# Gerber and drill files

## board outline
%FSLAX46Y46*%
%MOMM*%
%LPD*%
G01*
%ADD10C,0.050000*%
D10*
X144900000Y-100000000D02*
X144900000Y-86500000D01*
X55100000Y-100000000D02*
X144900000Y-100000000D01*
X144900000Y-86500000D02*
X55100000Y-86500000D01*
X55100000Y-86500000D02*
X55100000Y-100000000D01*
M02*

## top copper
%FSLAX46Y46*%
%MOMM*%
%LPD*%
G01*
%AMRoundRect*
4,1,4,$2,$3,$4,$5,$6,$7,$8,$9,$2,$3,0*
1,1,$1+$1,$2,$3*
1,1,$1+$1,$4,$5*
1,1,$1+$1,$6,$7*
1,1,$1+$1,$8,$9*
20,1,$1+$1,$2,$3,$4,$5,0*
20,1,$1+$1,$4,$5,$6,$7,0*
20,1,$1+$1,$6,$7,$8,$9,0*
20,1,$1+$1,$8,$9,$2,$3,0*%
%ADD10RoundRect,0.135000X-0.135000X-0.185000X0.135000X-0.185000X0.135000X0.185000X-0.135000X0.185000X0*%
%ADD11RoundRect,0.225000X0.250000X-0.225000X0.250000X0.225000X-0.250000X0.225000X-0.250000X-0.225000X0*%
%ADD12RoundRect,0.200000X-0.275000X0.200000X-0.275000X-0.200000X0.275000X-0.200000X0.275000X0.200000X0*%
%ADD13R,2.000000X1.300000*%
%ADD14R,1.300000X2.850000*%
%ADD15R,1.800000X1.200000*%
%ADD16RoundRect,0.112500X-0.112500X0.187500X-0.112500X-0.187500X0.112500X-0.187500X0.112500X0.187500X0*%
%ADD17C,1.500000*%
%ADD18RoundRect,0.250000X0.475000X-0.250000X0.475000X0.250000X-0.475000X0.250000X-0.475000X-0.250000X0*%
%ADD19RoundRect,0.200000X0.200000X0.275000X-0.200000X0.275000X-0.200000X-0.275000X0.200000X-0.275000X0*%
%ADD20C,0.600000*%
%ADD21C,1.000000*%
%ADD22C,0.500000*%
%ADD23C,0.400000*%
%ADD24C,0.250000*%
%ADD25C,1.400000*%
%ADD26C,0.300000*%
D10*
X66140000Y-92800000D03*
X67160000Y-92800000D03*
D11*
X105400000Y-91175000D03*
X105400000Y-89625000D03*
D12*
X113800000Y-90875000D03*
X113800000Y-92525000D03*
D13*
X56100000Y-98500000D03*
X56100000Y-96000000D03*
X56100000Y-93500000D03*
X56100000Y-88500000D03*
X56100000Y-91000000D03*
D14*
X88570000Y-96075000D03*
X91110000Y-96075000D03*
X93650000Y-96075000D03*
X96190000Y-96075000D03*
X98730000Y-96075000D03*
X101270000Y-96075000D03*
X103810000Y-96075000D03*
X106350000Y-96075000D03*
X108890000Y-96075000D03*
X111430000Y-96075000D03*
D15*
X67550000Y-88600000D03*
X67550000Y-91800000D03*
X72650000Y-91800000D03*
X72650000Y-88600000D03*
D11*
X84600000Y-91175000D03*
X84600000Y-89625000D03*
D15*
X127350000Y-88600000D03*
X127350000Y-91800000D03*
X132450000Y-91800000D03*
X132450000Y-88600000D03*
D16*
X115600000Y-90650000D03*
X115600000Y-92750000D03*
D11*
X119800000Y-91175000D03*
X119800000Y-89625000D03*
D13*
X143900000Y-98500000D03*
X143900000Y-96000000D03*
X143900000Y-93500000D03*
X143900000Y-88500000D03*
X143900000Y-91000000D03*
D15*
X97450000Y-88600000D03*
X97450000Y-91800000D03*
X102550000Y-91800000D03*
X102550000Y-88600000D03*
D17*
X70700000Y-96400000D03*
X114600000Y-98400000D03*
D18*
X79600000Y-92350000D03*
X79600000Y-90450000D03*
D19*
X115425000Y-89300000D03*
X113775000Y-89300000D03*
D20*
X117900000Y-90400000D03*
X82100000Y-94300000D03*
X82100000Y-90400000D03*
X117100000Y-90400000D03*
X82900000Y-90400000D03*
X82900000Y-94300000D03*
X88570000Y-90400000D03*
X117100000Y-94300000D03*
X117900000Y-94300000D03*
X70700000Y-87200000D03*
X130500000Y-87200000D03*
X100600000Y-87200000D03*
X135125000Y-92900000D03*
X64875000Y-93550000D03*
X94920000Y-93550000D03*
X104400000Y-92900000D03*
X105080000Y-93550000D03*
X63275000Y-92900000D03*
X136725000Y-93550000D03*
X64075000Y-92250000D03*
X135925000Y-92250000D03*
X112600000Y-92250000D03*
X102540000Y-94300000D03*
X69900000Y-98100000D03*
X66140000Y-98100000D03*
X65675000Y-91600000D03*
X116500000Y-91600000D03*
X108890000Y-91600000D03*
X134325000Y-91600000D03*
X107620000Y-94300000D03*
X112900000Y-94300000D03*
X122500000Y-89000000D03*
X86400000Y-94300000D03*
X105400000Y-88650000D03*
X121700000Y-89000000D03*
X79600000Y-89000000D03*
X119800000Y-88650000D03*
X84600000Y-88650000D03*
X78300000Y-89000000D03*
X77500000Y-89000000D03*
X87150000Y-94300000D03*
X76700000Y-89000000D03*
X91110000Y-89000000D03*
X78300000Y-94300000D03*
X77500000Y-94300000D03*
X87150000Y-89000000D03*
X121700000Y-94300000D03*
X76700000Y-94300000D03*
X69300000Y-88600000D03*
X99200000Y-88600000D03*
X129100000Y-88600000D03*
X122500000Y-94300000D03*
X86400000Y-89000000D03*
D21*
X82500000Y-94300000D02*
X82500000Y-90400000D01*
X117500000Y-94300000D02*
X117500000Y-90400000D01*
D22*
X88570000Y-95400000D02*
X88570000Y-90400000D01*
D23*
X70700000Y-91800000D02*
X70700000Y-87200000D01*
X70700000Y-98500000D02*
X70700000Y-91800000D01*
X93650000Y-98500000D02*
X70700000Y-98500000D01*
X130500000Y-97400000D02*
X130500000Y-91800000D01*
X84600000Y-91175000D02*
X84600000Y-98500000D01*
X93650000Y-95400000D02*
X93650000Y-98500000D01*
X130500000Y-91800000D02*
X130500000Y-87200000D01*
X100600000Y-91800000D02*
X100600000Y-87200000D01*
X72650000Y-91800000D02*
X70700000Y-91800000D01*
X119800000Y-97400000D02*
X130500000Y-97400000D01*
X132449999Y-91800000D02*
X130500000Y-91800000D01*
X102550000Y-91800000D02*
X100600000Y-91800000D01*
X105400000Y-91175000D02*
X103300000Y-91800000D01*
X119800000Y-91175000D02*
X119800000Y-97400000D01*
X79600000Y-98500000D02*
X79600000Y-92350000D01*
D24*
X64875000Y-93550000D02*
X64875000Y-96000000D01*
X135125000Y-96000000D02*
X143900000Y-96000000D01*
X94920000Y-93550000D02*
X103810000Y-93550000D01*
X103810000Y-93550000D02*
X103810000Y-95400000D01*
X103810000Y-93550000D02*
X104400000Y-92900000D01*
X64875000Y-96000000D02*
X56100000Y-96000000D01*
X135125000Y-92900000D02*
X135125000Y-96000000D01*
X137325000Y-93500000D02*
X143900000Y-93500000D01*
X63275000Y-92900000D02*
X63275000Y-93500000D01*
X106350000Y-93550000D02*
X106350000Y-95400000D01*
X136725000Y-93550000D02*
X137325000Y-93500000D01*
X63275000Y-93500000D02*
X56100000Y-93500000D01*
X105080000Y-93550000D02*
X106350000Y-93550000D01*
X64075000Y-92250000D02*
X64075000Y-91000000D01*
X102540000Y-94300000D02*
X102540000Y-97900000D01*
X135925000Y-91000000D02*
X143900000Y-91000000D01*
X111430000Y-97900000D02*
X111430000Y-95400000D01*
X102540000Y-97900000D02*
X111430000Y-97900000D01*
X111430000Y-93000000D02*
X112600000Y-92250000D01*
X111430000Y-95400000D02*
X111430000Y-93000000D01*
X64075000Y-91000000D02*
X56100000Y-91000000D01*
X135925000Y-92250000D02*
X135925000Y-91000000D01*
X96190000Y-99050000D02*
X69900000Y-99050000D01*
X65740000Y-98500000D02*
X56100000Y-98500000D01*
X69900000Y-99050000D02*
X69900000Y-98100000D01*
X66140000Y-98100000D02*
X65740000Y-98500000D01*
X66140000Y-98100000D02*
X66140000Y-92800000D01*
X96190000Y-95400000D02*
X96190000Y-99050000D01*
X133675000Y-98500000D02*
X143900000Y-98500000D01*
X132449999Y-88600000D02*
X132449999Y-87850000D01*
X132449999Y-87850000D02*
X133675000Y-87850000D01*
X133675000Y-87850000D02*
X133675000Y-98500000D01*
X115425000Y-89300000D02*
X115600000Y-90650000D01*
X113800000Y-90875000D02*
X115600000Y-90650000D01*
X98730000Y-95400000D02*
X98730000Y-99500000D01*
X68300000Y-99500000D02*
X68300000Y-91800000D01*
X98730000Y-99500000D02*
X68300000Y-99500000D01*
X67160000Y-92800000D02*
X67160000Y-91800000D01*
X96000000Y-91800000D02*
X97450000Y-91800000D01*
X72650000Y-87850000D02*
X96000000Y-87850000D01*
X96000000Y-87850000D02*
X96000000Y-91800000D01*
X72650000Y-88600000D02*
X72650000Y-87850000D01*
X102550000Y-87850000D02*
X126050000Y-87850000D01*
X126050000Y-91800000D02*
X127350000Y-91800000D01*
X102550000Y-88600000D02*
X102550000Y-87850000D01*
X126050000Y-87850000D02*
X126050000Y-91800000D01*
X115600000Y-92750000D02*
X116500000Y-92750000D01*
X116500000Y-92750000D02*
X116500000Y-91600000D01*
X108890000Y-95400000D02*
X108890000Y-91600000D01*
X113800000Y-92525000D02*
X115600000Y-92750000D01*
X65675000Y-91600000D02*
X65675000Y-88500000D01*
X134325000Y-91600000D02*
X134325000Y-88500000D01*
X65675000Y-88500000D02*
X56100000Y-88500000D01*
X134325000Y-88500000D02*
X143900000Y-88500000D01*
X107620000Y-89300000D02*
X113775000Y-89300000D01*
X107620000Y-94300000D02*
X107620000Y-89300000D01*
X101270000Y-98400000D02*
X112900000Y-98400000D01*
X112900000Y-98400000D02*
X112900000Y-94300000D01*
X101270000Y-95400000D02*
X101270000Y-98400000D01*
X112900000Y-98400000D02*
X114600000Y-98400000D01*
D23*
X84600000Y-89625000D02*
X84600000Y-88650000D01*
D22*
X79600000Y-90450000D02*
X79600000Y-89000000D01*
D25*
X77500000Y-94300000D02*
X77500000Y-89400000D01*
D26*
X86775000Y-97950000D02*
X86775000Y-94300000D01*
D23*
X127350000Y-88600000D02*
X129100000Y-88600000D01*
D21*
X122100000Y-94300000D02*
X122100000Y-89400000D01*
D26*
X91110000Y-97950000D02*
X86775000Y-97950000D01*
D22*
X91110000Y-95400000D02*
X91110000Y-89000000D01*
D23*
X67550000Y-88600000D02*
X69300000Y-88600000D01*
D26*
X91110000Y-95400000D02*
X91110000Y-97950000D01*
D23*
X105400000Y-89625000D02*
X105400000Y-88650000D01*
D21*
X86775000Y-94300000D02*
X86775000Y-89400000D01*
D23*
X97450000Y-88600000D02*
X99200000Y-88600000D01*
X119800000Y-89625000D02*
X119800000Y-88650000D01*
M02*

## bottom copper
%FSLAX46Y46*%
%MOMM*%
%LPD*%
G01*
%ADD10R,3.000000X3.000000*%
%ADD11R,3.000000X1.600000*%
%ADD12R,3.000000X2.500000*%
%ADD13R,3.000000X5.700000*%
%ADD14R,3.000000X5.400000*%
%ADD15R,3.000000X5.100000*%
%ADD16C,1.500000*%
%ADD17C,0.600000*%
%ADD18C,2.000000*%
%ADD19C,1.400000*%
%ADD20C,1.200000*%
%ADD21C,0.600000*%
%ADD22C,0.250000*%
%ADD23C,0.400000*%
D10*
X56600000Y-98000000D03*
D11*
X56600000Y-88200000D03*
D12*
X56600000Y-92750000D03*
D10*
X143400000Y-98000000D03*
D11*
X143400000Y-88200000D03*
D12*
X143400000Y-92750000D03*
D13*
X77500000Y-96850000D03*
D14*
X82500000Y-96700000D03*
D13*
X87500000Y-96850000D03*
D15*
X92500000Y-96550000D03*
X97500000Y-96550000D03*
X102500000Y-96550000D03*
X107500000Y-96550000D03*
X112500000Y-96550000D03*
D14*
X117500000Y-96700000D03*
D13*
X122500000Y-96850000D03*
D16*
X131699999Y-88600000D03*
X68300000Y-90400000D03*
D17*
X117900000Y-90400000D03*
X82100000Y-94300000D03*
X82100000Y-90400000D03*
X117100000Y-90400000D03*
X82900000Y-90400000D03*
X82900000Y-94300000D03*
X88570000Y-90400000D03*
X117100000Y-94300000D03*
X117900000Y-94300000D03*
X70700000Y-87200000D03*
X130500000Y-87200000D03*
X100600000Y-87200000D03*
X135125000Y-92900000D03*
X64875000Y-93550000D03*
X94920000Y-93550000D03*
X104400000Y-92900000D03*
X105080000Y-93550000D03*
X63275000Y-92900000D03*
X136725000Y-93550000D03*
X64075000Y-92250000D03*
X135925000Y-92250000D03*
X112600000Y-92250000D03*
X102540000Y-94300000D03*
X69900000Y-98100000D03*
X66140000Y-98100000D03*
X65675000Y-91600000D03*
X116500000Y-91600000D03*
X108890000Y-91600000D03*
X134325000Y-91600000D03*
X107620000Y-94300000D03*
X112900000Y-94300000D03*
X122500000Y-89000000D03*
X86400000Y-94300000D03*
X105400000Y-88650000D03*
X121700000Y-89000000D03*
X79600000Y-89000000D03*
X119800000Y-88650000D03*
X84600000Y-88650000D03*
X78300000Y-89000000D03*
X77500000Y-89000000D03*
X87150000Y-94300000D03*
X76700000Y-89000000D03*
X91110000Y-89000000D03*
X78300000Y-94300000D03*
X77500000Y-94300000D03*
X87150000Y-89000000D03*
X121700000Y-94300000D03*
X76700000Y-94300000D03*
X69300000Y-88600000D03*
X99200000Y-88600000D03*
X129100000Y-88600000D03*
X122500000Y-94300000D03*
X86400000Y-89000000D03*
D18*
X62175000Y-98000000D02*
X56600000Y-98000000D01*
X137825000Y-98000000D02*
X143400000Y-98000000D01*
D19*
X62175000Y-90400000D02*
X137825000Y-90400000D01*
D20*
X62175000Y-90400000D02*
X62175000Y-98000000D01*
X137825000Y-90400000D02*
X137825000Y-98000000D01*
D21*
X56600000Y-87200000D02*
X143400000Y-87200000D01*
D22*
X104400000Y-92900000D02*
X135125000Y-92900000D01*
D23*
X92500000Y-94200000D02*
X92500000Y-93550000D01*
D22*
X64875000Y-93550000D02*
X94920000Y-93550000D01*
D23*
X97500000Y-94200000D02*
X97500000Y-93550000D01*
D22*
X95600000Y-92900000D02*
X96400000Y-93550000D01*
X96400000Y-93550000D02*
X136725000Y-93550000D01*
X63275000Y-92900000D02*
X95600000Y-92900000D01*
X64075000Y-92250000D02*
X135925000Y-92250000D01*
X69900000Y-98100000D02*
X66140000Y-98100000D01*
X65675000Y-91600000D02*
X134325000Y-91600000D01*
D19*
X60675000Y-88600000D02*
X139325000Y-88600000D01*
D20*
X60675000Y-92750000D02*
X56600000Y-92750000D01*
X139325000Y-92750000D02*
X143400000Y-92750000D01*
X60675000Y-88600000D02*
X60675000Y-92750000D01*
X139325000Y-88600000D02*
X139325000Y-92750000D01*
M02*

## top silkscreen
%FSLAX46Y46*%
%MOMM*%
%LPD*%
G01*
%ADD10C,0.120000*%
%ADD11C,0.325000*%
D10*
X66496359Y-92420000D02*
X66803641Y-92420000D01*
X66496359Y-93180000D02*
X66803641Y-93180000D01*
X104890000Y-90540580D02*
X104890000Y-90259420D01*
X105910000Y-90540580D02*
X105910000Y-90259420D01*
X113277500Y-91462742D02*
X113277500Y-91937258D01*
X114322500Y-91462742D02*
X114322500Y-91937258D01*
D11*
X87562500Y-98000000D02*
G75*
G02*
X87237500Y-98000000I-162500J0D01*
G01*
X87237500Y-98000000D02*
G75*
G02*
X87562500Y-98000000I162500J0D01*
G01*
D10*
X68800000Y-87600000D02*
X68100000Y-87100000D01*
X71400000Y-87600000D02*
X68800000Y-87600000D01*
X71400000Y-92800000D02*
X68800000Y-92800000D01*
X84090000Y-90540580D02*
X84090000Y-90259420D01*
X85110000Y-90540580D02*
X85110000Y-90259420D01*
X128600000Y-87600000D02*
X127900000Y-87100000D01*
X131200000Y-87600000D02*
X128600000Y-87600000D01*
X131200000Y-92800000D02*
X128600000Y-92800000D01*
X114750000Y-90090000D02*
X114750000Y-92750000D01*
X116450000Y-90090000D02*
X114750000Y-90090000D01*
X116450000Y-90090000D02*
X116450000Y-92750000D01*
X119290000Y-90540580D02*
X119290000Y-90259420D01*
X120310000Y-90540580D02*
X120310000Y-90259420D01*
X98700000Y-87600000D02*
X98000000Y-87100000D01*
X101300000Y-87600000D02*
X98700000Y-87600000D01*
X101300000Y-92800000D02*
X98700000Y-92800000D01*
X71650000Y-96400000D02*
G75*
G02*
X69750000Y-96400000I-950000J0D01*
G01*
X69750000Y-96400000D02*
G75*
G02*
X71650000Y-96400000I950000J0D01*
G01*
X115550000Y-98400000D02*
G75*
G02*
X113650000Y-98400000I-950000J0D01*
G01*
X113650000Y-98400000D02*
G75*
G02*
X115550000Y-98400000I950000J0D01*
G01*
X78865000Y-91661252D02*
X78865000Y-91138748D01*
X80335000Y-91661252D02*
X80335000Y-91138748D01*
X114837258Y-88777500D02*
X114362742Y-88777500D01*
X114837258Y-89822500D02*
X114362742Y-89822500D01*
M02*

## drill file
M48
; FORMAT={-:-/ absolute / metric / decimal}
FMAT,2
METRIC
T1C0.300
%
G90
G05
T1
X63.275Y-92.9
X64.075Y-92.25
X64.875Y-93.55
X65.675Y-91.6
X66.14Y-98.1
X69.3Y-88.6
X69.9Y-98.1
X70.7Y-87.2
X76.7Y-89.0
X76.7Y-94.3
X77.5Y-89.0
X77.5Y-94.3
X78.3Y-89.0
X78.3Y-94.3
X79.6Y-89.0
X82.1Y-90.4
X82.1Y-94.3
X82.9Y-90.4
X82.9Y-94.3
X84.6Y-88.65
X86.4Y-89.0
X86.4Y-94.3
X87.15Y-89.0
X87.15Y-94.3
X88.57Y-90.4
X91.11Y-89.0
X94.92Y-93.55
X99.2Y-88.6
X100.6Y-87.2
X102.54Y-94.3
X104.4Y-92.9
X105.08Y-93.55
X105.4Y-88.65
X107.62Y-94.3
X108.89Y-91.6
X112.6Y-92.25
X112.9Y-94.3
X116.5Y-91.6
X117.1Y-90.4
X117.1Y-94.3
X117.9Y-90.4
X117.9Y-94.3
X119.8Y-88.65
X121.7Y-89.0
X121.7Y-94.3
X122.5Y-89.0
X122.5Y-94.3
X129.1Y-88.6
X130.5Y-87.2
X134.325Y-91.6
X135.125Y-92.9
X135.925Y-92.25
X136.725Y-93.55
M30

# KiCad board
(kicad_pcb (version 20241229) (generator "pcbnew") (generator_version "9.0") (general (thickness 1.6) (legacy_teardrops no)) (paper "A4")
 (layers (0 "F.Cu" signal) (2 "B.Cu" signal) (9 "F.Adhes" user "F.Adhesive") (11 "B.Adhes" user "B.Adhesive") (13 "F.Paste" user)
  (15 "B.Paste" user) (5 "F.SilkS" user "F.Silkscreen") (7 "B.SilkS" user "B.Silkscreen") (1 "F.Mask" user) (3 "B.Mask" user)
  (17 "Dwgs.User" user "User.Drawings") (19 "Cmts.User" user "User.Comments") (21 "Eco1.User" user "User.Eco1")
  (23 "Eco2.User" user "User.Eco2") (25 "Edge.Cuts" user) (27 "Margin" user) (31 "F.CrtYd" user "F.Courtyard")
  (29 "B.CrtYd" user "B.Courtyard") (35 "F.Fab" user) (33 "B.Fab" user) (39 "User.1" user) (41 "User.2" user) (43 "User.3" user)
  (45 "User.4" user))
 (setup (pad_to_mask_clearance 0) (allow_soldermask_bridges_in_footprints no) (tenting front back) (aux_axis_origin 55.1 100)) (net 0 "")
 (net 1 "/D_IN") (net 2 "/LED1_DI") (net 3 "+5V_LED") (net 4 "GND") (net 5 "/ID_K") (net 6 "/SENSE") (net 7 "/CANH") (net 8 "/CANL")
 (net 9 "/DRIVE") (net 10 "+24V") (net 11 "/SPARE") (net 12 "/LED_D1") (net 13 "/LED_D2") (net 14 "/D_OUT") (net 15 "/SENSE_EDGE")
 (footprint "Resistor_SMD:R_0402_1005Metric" (layer "F.Cu") (at 66.65 92.8)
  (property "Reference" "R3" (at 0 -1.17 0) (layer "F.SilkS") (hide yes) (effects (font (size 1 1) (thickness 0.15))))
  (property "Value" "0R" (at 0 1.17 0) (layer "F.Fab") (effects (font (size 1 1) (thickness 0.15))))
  (fp_line (start -0.153641 -0.38) (end 0.153641 -0.38) (stroke (width 0.12) (type solid)) (layer "F.SilkS"))
  (fp_line (start -0.153641 0.38) (end 0.153641 0.38) (stroke (width 0.12) (type solid)) (layer "F.SilkS"))
  (pad "1" smd roundrect (at -0.51 0) (size 0.54 0.64) (layers "F.Cu" "F.Mask" "F.Paste") (roundrect_rratio 0.25) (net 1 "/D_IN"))
  (pad "2" smd roundrect (at 0.51 0) (size 0.54 0.64) (layers "F.Cu" "F.Mask" "F.Paste") (roundrect_rratio 0.25) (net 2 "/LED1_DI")))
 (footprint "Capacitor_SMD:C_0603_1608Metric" (layer "F.Cu") (at 105.4 90.4 90)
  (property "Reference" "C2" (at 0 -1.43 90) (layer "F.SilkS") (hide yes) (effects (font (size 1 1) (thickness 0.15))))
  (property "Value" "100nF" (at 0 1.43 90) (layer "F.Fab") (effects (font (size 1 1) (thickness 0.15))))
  (fp_line (start -0.14058 -0.51) (end 0.14058 -0.51) (stroke (width 0.12) (type solid)) (layer "F.SilkS"))
  (fp_line (start -0.14058 0.51) (end 0.14058 0.51) (stroke (width 0.12) (type solid)) (layer "F.SilkS"))
  (pad "1" smd roundrect (at -0.775 0 90) (size 0.9 0.95) (layers "F.Cu" "F.Mask" "F.Paste") (roundrect_rratio 0.25) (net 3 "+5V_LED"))
  (pad "2" smd roundrect (at 0.775 0 90) (size 0.9 0.95) (layers "F.Cu" "F.Mask" "F.Paste") (roundrect_rratio 0.25) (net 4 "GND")))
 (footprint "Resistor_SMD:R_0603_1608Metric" (layer "F.Cu") (at 113.8 91.7 -90)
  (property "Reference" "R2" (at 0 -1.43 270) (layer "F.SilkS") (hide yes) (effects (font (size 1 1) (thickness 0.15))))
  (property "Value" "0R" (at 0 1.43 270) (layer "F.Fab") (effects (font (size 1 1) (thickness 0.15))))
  (fp_line (start -0.237258 0.5225) (end 0.237258 0.5225) (stroke (width 0.12) (type solid)) (layer "F.SilkS"))
  (fp_line (start -0.237258 -0.5225) (end 0.237258 -0.5225) (stroke (width 0.12) (type solid)) (layer "F.SilkS"))
  (pad "1" smd roundrect (at -0.825 0 270) (size 0.8 0.95) (layers "F.Cu" "F.Mask" "F.Paste") (roundrect_rratio 0.25) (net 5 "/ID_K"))
  (pad "2" smd roundrect (at 0.825 0 270) (size 0.8 0.95) (layers "F.Cu" "F.Mask" "F.Paste") (roundrect_rratio 0.25) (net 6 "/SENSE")))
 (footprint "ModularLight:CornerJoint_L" (layer "F.Cu") (at 55.1 100)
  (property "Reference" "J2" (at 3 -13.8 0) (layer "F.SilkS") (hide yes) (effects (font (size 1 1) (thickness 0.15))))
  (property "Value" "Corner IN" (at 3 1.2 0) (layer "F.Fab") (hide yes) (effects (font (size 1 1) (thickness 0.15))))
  (pad "1" smd rect (at 1 -1.5) (size 2 1.3) (layers "F.Cu" "F.Mask" "F.Paste") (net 1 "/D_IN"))
  (pad "2" smd rect (at 1 -4) (size 2 1.3) (layers "F.Cu" "F.Mask" "F.Paste") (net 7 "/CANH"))
  (pad "3" smd rect (at 1 -6.5) (size 2 1.3) (layers "F.Cu" "F.Mask" "F.Paste") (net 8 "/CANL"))
  (pad "4" smd rect (at 1 -11.5) (size 2 1.3) (layers "F.Cu" "F.Mask" "F.Paste") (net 6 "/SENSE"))
  (pad "5" smd rect (at 1 -9) (size 2 1.3) (layers "F.Cu" "F.Mask" "F.Paste") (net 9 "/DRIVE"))
  (pad "6" smd rect (at 1.5 -2) (size 3 3) (layers "B.Cu" "B.Mask") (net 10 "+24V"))
  (pad "7" smd rect (at 1.5 -11.8) (size 3 1.6) (layers "B.Cu" "B.Mask") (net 3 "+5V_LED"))
  (pad "8" smd rect (at 1.5 -7.25) (size 3 2.5) (layers "B.Cu" "B.Mask") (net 4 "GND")))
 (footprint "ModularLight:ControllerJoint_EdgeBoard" (layer "F.Cu") (at 100 94.75)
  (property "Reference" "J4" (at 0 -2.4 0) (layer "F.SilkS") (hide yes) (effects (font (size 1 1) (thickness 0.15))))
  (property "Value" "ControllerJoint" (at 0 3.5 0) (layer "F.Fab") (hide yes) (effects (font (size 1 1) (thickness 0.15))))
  (fp_circle (center -12.6 3.25) (end -12.35 3.25) (stroke (width 0.15) (type solid)) (fill yes) (layer "F.SilkS"))
  (pad "1" smd rect (at -11.43 1.325) (size 1.3 2.85) (layers "F.Cu" "F.Mask" "F.Paste") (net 10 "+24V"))
  (pad "2" smd rect (at -8.89 1.325) (size 1.3 2.85) (layers "F.Cu" "F.Mask" "F.Paste") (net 4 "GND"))
  (pad "3" smd rect (at -6.35 1.325) (size 1.3 2.85) (layers "F.Cu" "F.Mask" "F.Paste") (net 3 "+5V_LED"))
  (pad "4" smd rect (at -3.81 1.325) (size 1.3 2.85) (layers "F.Cu" "F.Mask" "F.Paste") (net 1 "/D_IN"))
  (pad "5" smd rect (at -1.27 1.325) (size 1.3 2.85) (layers "F.Cu" "F.Mask" "F.Paste") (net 2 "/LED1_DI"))
  (pad "6" smd rect (at 1.27 1.325) (size 1.3 2.85) (layers "F.Cu" "F.Mask" "F.Paste") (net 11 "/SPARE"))
  (pad "7" smd rect (at 3.81 1.325) (size 1.3 2.85) (layers "F.Cu" "F.Mask" "F.Paste") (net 7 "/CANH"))
  (pad "8" smd rect (at 6.35 1.325) (size 1.3 2.85) (layers "F.Cu" "F.Mask" "F.Paste") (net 8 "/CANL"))
  (pad "9" smd rect (at 8.89 1.325) (size 1.3 2.85) (layers "F.Cu" "F.Mask" "F.Paste") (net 6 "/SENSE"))
  (pad "10" smd rect (at 11.43 1.325) (size 1.3 2.85) (layers "F.Cu" "F.Mask" "F.Paste") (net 9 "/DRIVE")))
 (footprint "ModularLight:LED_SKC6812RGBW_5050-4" (layer "F.Cu") (at 70.1 90.2 180)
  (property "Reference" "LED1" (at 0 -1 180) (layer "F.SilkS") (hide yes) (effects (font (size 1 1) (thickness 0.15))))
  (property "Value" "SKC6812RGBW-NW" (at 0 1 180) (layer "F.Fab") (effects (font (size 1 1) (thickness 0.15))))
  (fp_line (start 1.3 2.6) (end 2 3.1) (stroke (width 0.12) (type solid)) (layer "F.SilkS"))
  (fp_line (start -1.3 2.6) (end 1.3 2.6) (stroke (width 0.12) (type solid)) (layer "F.SilkS"))
  (fp_line (start -1.3 -2.6) (end 1.3 -2.6) (stroke (width 0.12) (type solid)) (layer "F.SilkS"))
  (pad "1" smd rect (at 2.55 1.6 180) (size 1.8 1.2) (layers "F.Cu" "F.Mask" "F.Paste") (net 4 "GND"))
  (pad "2" smd rect (at 2.55 -1.6 180) (size 1.8 1.2) (layers "F.Cu" "F.Mask" "F.Paste") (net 2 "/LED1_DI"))
  (pad "3" smd rect (at -2.55 -1.6 180) (size 1.8 1.2) (layers "F.Cu" "F.Mask" "F.Paste") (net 3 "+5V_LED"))
  (pad "4" smd rect (at -2.55 1.6 180) (size 1.8 1.2) (layers "F.Cu" "F.Mask" "F.Paste") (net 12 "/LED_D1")))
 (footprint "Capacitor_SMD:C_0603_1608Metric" (layer "F.Cu") (at 84.6 90.4 90)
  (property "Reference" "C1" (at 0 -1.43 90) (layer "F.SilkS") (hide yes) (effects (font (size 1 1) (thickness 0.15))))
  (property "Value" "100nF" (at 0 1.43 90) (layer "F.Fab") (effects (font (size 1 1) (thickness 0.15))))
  (fp_line (start -0.14058 -0.51) (end 0.14058 -0.51) (stroke (width 0.12) (type solid)) (layer "F.SilkS"))
  (fp_line (start -0.14058 0.51) (end 0.14058 0.51) (stroke (width 0.12) (type solid)) (layer "F.SilkS"))
  (pad "1" smd roundrect (at -0.775 0 90) (size 0.9 0.95) (layers "F.Cu" "F.Mask" "F.Paste") (roundrect_rratio 0.25) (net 3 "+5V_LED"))
  (pad "2" smd roundrect (at 0.775 0 90) (size 0.9 0.95) (layers "F.Cu" "F.Mask" "F.Paste") (roundrect_rratio 0.25) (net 4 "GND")))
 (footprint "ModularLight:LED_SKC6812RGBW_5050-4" (layer "F.Cu") (at 129.9 90.2 180)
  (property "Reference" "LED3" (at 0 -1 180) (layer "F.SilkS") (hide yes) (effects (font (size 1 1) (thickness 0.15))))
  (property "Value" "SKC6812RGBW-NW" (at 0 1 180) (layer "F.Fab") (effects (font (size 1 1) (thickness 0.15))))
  (fp_line (start 1.3 2.6) (end 2 3.1) (stroke (width 0.12) (type solid)) (layer "F.SilkS"))
  (fp_line (start -1.3 2.6) (end 1.3 2.6) (stroke (width 0.12) (type solid)) (layer "F.SilkS"))
  (fp_line (start -1.3 -2.6) (end 1.3 -2.6) (stroke (width 0.12) (type solid)) (layer "F.SilkS"))
  (pad "1" smd rect (at 2.55 1.6 180) (size 1.8 1.2) (layers "F.Cu" "F.Mask" "F.Paste") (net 4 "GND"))
  (pad "2" smd rect (at 2.55 -1.6 180) (size 1.8 1.2) (layers "F.Cu" "F.Mask" "F.Paste") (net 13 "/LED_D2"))
  (pad "3" smd rect (at -2.55 -1.6 180) (size 1.8 1.2) (layers "F.Cu" "F.Mask" "F.Paste") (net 3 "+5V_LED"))
  (pad "4" smd rect (at -2.55 1.6 180) (size 1.8 1.2) (layers "F.Cu" "F.Mask" "F.Paste") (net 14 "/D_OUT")))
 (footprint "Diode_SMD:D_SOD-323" (layer "F.Cu") (at 115.6 91.7 -90)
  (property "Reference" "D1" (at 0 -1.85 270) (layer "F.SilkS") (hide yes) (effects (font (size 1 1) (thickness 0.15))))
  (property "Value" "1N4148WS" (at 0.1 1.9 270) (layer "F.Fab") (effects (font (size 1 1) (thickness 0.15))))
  (fp_line (start -1.61 0.85) (end 1.05 0.85) (stroke (width 0.12) (type solid)) (layer "F.SilkS"))
  (fp_line (start -1.61 -0.85) (end -1.61 0.85) (stroke (width 0.12) (type solid)) (layer "F.SilkS"))
  (fp_line (start -1.61 -0.85) (end 1.05 -0.85) (stroke (width 0.12) (type solid)) (layer "F.SilkS"))
  (pad "1" smd roundrect (at -1.05 0 270) (size 0.6 0.45) (layers "F.Cu" "F.Mask" "F.Paste") (roundrect_rratio 0.25) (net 5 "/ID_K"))
  (pad "2" smd roundrect (at 1.05 0 270) (size 0.6 0.45) (layers "F.Cu" "F.Mask" "F.Paste") (roundrect_rratio 0.25) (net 6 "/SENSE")))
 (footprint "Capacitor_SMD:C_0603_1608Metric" (layer "F.Cu") (at 119.8 90.4 90)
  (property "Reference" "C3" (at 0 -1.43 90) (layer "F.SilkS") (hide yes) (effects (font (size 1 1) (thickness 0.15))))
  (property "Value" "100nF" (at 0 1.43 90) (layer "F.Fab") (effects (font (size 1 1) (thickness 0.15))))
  (fp_line (start -0.14058 -0.51) (end 0.14058 -0.51) (stroke (width 0.12) (type solid)) (layer "F.SilkS"))
  (fp_line (start -0.14058 0.51) (end 0.14058 0.51) (stroke (width 0.12) (type solid)) (layer "F.SilkS"))
  (pad "1" smd roundrect (at -0.775 0 90) (size 0.9 0.95) (layers "F.Cu" "F.Mask" "F.Paste") (roundrect_rratio 0.25) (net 3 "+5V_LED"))
  (pad "2" smd roundrect (at 0.775 0 90) (size 0.9 0.95) (layers "F.Cu" "F.Mask" "F.Paste") (roundrect_rratio 0.25) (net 4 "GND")))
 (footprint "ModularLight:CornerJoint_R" (layer "F.Cu") (at 144.9 100)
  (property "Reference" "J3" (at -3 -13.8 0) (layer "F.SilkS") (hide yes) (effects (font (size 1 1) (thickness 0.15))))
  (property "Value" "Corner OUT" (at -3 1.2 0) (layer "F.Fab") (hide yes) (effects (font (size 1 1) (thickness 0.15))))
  (pad "1" smd rect (at -1 -1.5) (size 2 1.3) (layers "F.Cu" "F.Mask" "F.Paste") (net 14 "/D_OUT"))
  (pad "2" smd rect (at -1 -4) (size 2 1.3) (layers "F.Cu" "F.Mask" "F.Paste") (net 7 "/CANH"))
  (pad "3" smd rect (at -1 -6.5) (size 2 1.3) (layers "F.Cu" "F.Mask" "F.Paste") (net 8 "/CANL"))
  (pad "4" smd rect (at -1 -11.5) (size 2 1.3) (layers "F.Cu" "F.Mask" "F.Paste") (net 6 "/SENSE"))
  (pad "5" smd rect (at -1 -9) (size 2 1.3) (layers "F.Cu" "F.Mask" "F.Paste") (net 9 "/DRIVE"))
  (pad "6" smd rect (at -1.5 -2) (size 3 3) (layers "B.Cu" "B.Mask") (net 10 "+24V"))
  (pad "7" smd rect (at -1.5 -11.8) (size 3 1.6) (layers "B.Cu" "B.Mask") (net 3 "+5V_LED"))
  (pad "8" smd rect (at -1.5 -7.25) (size 3 2.5) (layers "B.Cu" "B.Mask") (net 4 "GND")))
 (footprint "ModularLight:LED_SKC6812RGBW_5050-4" (layer "F.Cu") (at 100 90.2 180)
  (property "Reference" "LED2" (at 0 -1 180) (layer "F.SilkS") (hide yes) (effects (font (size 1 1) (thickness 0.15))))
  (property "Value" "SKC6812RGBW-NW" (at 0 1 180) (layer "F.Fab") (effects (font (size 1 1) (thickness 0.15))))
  (fp_line (start 1.3 2.6) (end 2 3.1) (stroke (width 0.12) (type solid)) (layer "F.SilkS"))
  (fp_line (start -1.3 2.6) (end 1.3 2.6) (stroke (width 0.12) (type solid)) (layer "F.SilkS"))
  (fp_line (start -1.3 -2.6) (end 1.3 -2.6) (stroke (width 0.12) (type solid)) (layer "F.SilkS"))
  (pad "1" smd rect (at 2.55 1.6 180) (size 1.8 1.2) (layers "F.Cu" "F.Mask" "F.Paste") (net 4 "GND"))
  (pad "2" smd rect (at 2.55 -1.6 180) (size 1.8 1.2) (layers "F.Cu" "F.Mask" "F.Paste") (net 12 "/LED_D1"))
  (pad "3" smd rect (at -2.55 -1.6 180) (size 1.8 1.2) (layers "F.Cu" "F.Mask" "F.Paste") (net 3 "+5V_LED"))
  (pad "4" smd rect (at -2.55 1.6 180) (size 1.8 1.2) (layers "F.Cu" "F.Mask" "F.Paste") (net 13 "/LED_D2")))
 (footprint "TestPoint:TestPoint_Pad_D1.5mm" (layer "F.Cu") (at 70.7 96.4)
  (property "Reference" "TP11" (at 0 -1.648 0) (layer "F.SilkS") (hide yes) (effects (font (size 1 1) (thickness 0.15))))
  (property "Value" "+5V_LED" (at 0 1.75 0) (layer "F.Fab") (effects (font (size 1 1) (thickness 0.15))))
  (fp_circle (center 0 0) (end 0 0.95) (stroke (width 0.12) (type solid)) (fill no) (layer "F.SilkS"))
  (pad "1" smd circle (at 0 0) (size 1.5 1.5) (layers "F.Cu" "F.Mask") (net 3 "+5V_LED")))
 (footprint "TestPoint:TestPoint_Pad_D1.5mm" (layer "F.Cu") (at 114.6 98.4)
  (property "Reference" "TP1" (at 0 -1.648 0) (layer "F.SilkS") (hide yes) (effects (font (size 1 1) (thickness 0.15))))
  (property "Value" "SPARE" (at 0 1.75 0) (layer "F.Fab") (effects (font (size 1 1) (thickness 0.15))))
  (fp_circle (center 0 0) (end 0 0.95) (stroke (width 0.12) (type solid)) (fill no) (layer "F.SilkS"))
  (pad "1" smd circle (at 0 0) (size 1.5 1.5) (layers "F.Cu" "F.Mask") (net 11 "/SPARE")))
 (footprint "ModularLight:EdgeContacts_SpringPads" (layer "F.Cu") (at 100 100)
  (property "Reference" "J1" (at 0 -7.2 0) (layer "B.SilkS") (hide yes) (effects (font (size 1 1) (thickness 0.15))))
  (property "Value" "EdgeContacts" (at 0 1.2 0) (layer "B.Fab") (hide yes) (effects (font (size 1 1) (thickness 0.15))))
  (pad "X1" smd rect (at -22.5 -3.15) (size 3 5.7) (layers "B.Cu" "B.Mask") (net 4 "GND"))
  (pad "X2" smd rect (at -17.5 -3.3) (size 3 5.4) (layers "B.Cu" "B.Mask") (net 10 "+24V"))
  (pad "X3" smd rect (at -12.5 -3.15) (size 3 5.7) (layers "B.Cu" "B.Mask") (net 4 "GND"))
  (pad "X4" smd rect (at -7.5 -3.45) (size 3 5.1) (layers "B.Cu" "B.Mask") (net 7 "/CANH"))
  (pad "X5" smd rect (at -2.5 -3.45) (size 3 5.1) (layers "B.Cu" "B.Mask") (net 8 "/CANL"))
  (pad "X6" smd rect (at 2.5 -3.45) (size 3 5.1) (layers "B.Cu" "B.Mask") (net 9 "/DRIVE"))
  (pad "X7" smd rect (at 7.5 -3.45) (size 3 5.1) (layers "B.Cu" "B.Mask") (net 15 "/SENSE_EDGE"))
  (pad "X8" smd rect (at 12.5 -3.45) (size 3 5.1) (layers "B.Cu" "B.Mask") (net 11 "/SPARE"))
  (pad "X9" smd rect (at 17.5 -3.3) (size 3 5.4) (layers "B.Cu" "B.Mask") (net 10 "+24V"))
  (pad "X10" smd rect (at 22.5 -3.15) (size 3 5.7) (layers "B.Cu" "B.Mask") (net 4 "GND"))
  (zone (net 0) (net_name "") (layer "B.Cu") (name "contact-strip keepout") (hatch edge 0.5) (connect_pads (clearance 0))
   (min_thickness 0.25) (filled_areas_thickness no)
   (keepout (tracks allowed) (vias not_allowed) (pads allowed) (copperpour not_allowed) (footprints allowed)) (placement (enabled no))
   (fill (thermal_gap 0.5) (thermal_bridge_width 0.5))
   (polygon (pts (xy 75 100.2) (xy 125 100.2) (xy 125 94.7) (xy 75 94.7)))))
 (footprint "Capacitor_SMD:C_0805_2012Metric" (layer "F.Cu") (at 79.6 91.4 90)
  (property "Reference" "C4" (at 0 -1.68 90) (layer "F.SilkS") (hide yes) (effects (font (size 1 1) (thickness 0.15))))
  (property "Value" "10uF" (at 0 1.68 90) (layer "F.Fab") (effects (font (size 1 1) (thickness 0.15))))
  (fp_line (start -0.261252 -0.735) (end 0.261252 -0.735) (stroke (width 0.12) (type solid)) (layer "F.SilkS"))
  (fp_line (start -0.261252 0.735) (end 0.261252 0.735) (stroke (width 0.12) (type solid)) (layer "F.SilkS"))
  (pad "1" smd roundrect (at -0.95 0 90) (size 1 1.45) (layers "F.Cu" "F.Mask" "F.Paste") (roundrect_rratio 0.25) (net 3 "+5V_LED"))
  (pad "2" smd roundrect (at 0.95 0 90) (size 1 1.45) (layers "F.Cu" "F.Mask" "F.Paste") (roundrect_rratio 0.25) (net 4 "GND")))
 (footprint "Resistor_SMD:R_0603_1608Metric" (layer "F.Cu") (at 114.6 89.3 180)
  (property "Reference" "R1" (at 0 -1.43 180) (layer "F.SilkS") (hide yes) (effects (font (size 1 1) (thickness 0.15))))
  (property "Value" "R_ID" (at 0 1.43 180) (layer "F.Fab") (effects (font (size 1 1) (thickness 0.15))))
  (fp_line (start -0.237258 0.5225) (end 0.237258 0.5225) (stroke (width 0.12) (type solid)) (layer "F.SilkS"))
  (fp_line (start -0.237258 -0.5225) (end 0.237258 -0.5225) (stroke (width 0.12) (type solid)) (layer "F.SilkS"))
  (pad "1" smd roundrect (at -0.825 0 180) (size 0.8 0.95) (layers "F.Cu" "F.Mask" "F.Paste") (roundrect_rratio 0.25) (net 5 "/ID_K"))
  (pad "2" smd roundrect (at 0.825 0 180) (size 0.8 0.95) (layers "F.Cu" "F.Mask" "F.Paste") (roundrect_rratio 0.25) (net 15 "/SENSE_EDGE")))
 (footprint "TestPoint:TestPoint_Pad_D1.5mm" (layer "B.Cu") (at 131.699999 88.6 180)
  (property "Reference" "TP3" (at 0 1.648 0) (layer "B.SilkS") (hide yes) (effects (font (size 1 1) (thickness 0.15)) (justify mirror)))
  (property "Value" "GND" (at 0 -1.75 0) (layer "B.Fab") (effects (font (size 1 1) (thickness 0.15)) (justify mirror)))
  (pad "1" smd circle (at 0 0 180) (size 1.5 1.5) (layers "B.Cu" "B.Mask") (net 4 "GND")))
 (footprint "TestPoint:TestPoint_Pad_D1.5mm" (layer "B.Cu") (at 68.3 90.4 180)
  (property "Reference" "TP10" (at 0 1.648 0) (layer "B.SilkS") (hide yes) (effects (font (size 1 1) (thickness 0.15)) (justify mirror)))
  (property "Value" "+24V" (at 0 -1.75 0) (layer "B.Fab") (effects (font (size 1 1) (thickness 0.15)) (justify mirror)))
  (pad "1" smd circle (at 0 0 180) (size 1.5 1.5) (layers "B.Cu" "B.Mask") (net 10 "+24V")))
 (gr_line (start 144.9 100) (end 144.9 86.5) (stroke (width 0.05) (type default)) (layer "Edge.Cuts"))
 (gr_line (start 55.1 100) (end 144.9 100) (stroke (width 0.05) (type default)) (layer "Edge.Cuts"))
 (gr_line (start 144.9 86.5) (end 55.1 86.5) (stroke (width 0.05) (type default)) (layer "Edge.Cuts"))
 (gr_line (start 55.1 86.5) (end 55.1 100) (stroke (width 0.05) (type default)) (layer "Edge.Cuts"))
 (segment (start 82.5 94.3) (end 82.5 90.4) (width 1) (locked yes) (layer "F.Cu") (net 10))
 (segment (start 117.5 94.3) (end 117.5 90.4) (width 1) (locked yes) (layer "F.Cu") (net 10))
 (segment (start 88.57 95.4) (end 88.57 90.4) (width 0.5) (locked yes) (layer "F.Cu") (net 10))
 (via (at 117.9 90.4) (size 0.6) (drill 0.3) (layers "F.Cu" "B.Cu") (locked yes) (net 10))
 (via (at 82.1 94.3) (size 0.6) (drill 0.3) (layers "F.Cu" "B.Cu") (locked yes) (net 10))
 (via (at 82.1 90.4) (size 0.6) (drill 0.3) (layers "F.Cu" "B.Cu") (locked yes) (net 10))
 (via (at 117.1 90.4) (size 0.6) (drill 0.3) (layers "F.Cu" "B.Cu") (locked yes) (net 10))
 (via (at 82.9 90.4) (size 0.6) (drill 0.3) (layers "F.Cu" "B.Cu") (locked yes) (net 10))
 (via (at 82.9 94.3) (size 0.6) (drill 0.3) (layers "F.Cu" "B.Cu") (locked yes) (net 10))
 (via (at 88.57 90.4) (size 0.6) (drill 0.3) (layers "F.Cu" "B.Cu") (locked yes) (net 10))
 (via (at 117.1 94.3) (size 0.6) (drill 0.3) (layers "F.Cu" "B.Cu") (locked yes) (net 10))
 (via (at 117.9 94.3) (size 0.6) (drill 0.3) (layers "F.Cu" "B.Cu") (locked yes) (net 10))
 (segment (start 62.175 98) (end 56.6 98) (width 2) (locked yes) (layer "B.Cu") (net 10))
 (segment (start 137.825 98) (end 143.4 98) (width 2) (locked yes) (layer "B.Cu") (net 10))
 (segment (start 62.175 90.4) (end 137.825 90.4) (width 1.4) (locked yes) (layer "B.Cu") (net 10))
 (segment (start 62.175 90.4) (end 62.175 98) (width 1.2) (locked yes) (layer "B.Cu") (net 10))
 (segment (start 137.825 90.4) (end 137.825 98) (width 1.2) (locked yes) (layer "B.Cu") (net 10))
 (segment (start 70.7 91.8) (end 70.7 87.2) (width 0.4) (locked yes) (layer "F.Cu") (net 3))
 (segment (start 70.7 98.5) (end 70.7 91.8) (width 0.4) (locked yes) (layer "F.Cu") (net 3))
 (segment (start 93.65 98.5) (end 70.7 98.5) (width 0.4) (locked yes) (layer "F.Cu") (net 3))
 (segment (start 130.5 97.4) (end 130.5 91.8) (width 0.4) (locked yes) (layer "F.Cu") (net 3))
 (segment (start 84.6 91.175) (end 84.6 98.5) (width 0.4) (locked yes) (layer "F.Cu") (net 3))
 (segment (start 93.65 95.4) (end 93.65 98.5) (width 0.4) (locked yes) (layer "F.Cu") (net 3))
 (segment (start 130.5 91.8) (end 130.5 87.2) (width 0.4) (locked yes) (layer "F.Cu") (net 3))
 (segment (start 100.6 91.8) (end 100.6 87.2) (width 0.4) (locked yes) (layer "F.Cu") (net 3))
 (segment (start 72.65 91.8) (end 70.7 91.8) (width 0.4) (locked yes) (layer "F.Cu") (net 3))
 (segment (start 119.8 97.4) (end 130.5 97.4) (width 0.4) (locked yes) (layer "F.Cu") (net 3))
 (segment (start 132.449999 91.8) (end 130.5 91.8) (width 0.4) (locked yes) (layer "F.Cu") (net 3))
 (segment (start 102.55 91.8) (end 100.6 91.8) (width 0.4) (locked yes) (layer "F.Cu") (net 3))
 (segment (start 105.4 91.175) (end 103.3 91.8) (width 0.4) (locked yes) (layer "F.Cu") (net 3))
 (segment (start 119.8 91.175) (end 119.8 97.4) (width 0.4) (locked yes) (layer "F.Cu") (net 3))
 (segment (start 79.6 98.5) (end 79.6 92.35) (width 0.4) (locked yes) (layer "F.Cu") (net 3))
 (via (at 70.7 87.2) (size 0.6) (drill 0.3) (layers "F.Cu" "B.Cu") (locked yes) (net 3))
 (via (at 130.5 87.2) (size 0.6) (drill 0.3) (layers "F.Cu" "B.Cu") (locked yes) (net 3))
 (via (at 100.6 87.2) (size 0.6) (drill 0.3) (layers "F.Cu" "B.Cu") (locked yes) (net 3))
 (segment (start 56.6 87.2) (end 143.4 87.2) (width 0.6) (locked yes) (layer "B.Cu") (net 3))
 (segment (start 64.875 93.55) (end 64.875 96) (width 0.25) (locked yes) (layer "F.Cu") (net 7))
 (segment (start 135.125 96) (end 143.9 96) (width 0.25) (locked yes) (layer "F.Cu") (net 7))
 (segment (start 94.92 93.55) (end 103.81 93.55) (width 0.25) (locked yes) (layer "F.Cu") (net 7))
 (segment (start 103.81 93.55) (end 103.81 95.4) (width 0.25) (locked yes) (layer "F.Cu") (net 7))
 (segment (start 103.81 93.55) (end 104.4 92.9) (width 0.25) (locked yes) (layer "F.Cu") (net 7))
 (segment (start 64.875 96) (end 56.1 96) (width 0.25) (locked yes) (layer "F.Cu") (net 7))
 (segment (start 135.125 92.9) (end 135.125 96) (width 0.25) (locked yes) (layer "F.Cu") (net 7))
 (via (at 135.125 92.9) (size 0.6) (drill 0.3) (layers "F.Cu" "B.Cu") (locked yes) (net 7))
 (via (at 64.875 93.55) (size 0.6) (drill 0.3) (layers "F.Cu" "B.Cu") (locked yes) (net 7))
 (via (at 94.92 93.55) (size 0.6) (drill 0.3) (layers "F.Cu" "B.Cu") (locked yes) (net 7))
 (via (at 104.4 92.9) (size 0.6) (drill 0.3) (layers "F.Cu" "B.Cu") (locked yes) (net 7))
 (segment (start 104.4 92.9) (end 135.125 92.9) (width 0.25) (locked yes) (layer "B.Cu") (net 7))
 (segment (start 92.5 94.2) (end 92.5 93.55) (width 0.4) (locked yes) (layer "B.Cu") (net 7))
 (segment (start 64.875 93.55) (end 94.92 93.55) (width 0.25) (locked yes) (layer "B.Cu") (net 7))
 (segment (start 137.325 93.5) (end 143.9 93.5) (width 0.25) (locked yes) (layer "F.Cu") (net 8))
 (segment (start 63.275 92.9) (end 63.275 93.5) (width 0.25) (locked yes) (layer "F.Cu") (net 8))
 (segment (start 106.35 93.55) (end 106.35 95.4) (width 0.25) (locked yes) (layer "F.Cu") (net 8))
 (segment (start 136.725 93.55) (end 137.325 93.5) (width 0.25) (locked yes) (layer "F.Cu") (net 8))
 (segment (start 63.275 93.5) (end 56.1 93.5) (width 0.25) (locked yes) (layer "F.Cu") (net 8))
 (segment (start 105.08 93.55) (end 106.35 93.55) (width 0.25) (locked yes) (layer "F.Cu") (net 8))
 (via (at 105.08 93.55) (size 0.6) (drill 0.3) (layers "F.Cu" "B.Cu") (locked yes) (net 8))
 (via (at 63.275 92.9) (size 0.6) (drill 0.3) (layers "F.Cu" "B.Cu") (locked yes) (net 8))
 (via (at 136.725 93.55) (size 0.6) (drill 0.3) (layers "F.Cu" "B.Cu") (locked yes) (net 8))
 (segment (start 97.5 94.2) (end 97.5 93.55) (width 0.4) (locked yes) (layer "B.Cu") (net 8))
 (segment (start 95.6 92.9) (end 96.4 93.55) (width 0.25) (locked yes) (layer "B.Cu") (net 8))
 (segment (start 96.4 93.55) (end 136.725 93.55) (width 0.25) (locked yes) (layer "B.Cu") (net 8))
 (segment (start 63.275 92.9) (end 95.6 92.9) (width 0.25) (locked yes) (layer "B.Cu") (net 8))
 (segment (start 64.075 92.25) (end 64.075 91) (width 0.25) (locked yes) (layer "F.Cu") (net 9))
 (segment (start 102.54 94.3) (end 102.54 97.9) (width 0.25) (locked yes) (layer "F.Cu") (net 9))
 (segment (start 135.925 91) (end 143.9 91) (width 0.25) (locked yes) (layer "F.Cu") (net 9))
 (segment (start 111.43 97.9) (end 111.43 95.4) (width 0.25) (locked yes) (layer "F.Cu") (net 9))
 (segment (start 102.54 97.9) (end 111.43 97.9) (width 0.25) (locked yes) (layer "F.Cu") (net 9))
 (segment (start 111.43 93) (end 112.6 92.25) (width 0.25) (locked yes) (layer "F.Cu") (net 9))
 (segment (start 111.43 95.4) (end 111.43 93) (width 0.25) (locked yes) (layer "F.Cu") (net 9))
 (segment (start 64.075 91) (end 56.1 91) (width 0.25) (locked yes) (layer "F.Cu") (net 9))
 (segment (start 135.925 92.25) (end 135.925 91) (width 0.25) (locked yes) (layer "F.Cu") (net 9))
 (via (at 64.075 92.25) (size 0.6) (drill 0.3) (layers "F.Cu" "B.Cu") (locked yes) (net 9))
 (via (at 135.925 92.25) (size 0.6) (drill 0.3) (layers "F.Cu" "B.Cu") (locked yes) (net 9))
 (via (at 112.6 92.25) (size 0.6) (drill 0.3) (layers "F.Cu" "B.Cu") (locked yes) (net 9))
 (via (at 102.54 94.3) (size 0.6) (drill 0.3) (layers "F.Cu" "B.Cu") (locked yes) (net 9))
 (segment (start 64.075 92.25) (end 135.925 92.25) (width 0.25) (locked yes) (layer "B.Cu") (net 9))
 (segment (start 96.19 99.05) (end 69.9 99.05) (width 0.25) (locked yes) (layer "F.Cu") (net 1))
 (segment (start 65.74 98.5) (end 56.1 98.5) (width 0.25) (locked yes) (layer "F.Cu") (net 1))
 (segment (start 69.9 99.05) (end 69.9 98.1) (width 0.25) (locked yes) (layer "F.Cu") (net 1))
 (segment (start 66.14 98.1) (end 65.74 98.5) (width 0.25) (locked yes) (layer "F.Cu") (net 1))
 (segment (start 66.14 98.1) (end 66.14 92.8) (width 0.25) (locked yes) (layer "F.Cu") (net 1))
 (segment (start 96.19 95.4) (end 96.19 99.05) (width 0.25) (locked yes) (layer "F.Cu") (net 1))
 (via (at 69.9 98.1) (size 0.6) (drill 0.3) (layers "F.Cu" "B.Cu") (locked yes) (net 1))
 (via (at 66.14 98.1) (size 0.6) (drill 0.3) (layers "F.Cu" "B.Cu") (locked yes) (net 1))
 (segment (start 69.9 98.1) (end 66.14 98.1) (width 0.25) (locked yes) (layer "B.Cu") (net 1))
 (segment (start 133.675 98.5) (end 143.9 98.5) (width 0.25) (locked yes) (layer "F.Cu") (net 14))
 (segment (start 132.449999 88.6) (end 132.449999 87.85) (width 0.25) (locked yes) (layer "F.Cu") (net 14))
 (segment (start 132.449999 87.85) (end 133.675 87.85) (width 0.25) (locked yes) (layer "F.Cu") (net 14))
 (segment (start 133.675 87.85) (end 133.675 98.5) (width 0.25) (locked yes) (layer "F.Cu") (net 14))
 (segment (start 115.425 89.3) (end 115.6 90.65) (width 0.25) (locked yes) (layer "F.Cu") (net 5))
 (segment (start 113.8 90.875) (end 115.6 90.65) (width 0.25) (locked yes) (layer "F.Cu") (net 5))
 (segment (start 98.73 95.4) (end 98.73 99.5) (width 0.25) (locked yes) (layer "F.Cu") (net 2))
 (segment (start 68.3 99.5) (end 68.3 91.8) (width 0.25) (locked yes) (layer "F.Cu") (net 2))
 (segment (start 98.73 99.5) (end 68.3 99.5) (width 0.25) (locked yes) (layer "F.Cu") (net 2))
 (segment (start 67.16 92.8) (end 67.16 91.8) (width 0.25) (locked yes) (layer "F.Cu") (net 2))
 (segment (start 96 91.8) (end 97.45 91.8) (width 0.25) (locked yes) (layer "F.Cu") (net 12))
 (segment (start 72.65 87.85) (end 96 87.85) (width 0.25) (locked yes) (layer "F.Cu") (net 12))
 (segment (start 96 87.85) (end 96 91.8) (width 0.25) (locked yes) (layer "F.Cu") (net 12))
 (segment (start 72.65 88.6) (end 72.65 87.85) (width 0.25) (locked yes) (layer "F.Cu") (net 12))
 (segment (start 102.55 87.85) (end 126.05 87.85) (width 0.25) (locked yes) (layer "F.Cu") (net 13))
 (segment (start 126.05 91.8) (end 127.35 91.8) (width 0.25) (locked yes) (layer "F.Cu") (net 13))
 (segment (start 102.55 88.6) (end 102.55 87.85) (width 0.25) (locked yes) (layer "F.Cu") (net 13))
 (segment (start 126.05 87.85) (end 126.05 91.8) (width 0.25) (locked yes) (layer "F.Cu") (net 13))
 (segment (start 115.6 92.75) (end 116.5 92.75) (width 0.25) (locked yes) (layer "F.Cu") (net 6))
 (segment (start 116.5 92.75) (end 116.5 91.6) (width 0.25) (locked yes) (layer "F.Cu") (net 6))
 (segment (start 108.89 95.4) (end 108.89 91.6) (width 0.25) (locked yes) (layer "F.Cu") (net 6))
 (segment (start 113.8 92.525) (end 115.6 92.75) (width 0.25) (locked yes) (layer "F.Cu") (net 6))
 (segment (start 65.675 91.6) (end 65.675 88.5) (width 0.25) (locked yes) (layer "F.Cu") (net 6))
 (segment (start 134.325 91.6) (end 134.325 88.5) (width 0.25) (locked yes) (layer "F.Cu") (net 6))
 (segment (start 65.675 88.5) (end 56.1 88.5) (width 0.25) (locked yes) (layer "F.Cu") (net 6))
 (segment (start 134.325 88.5) (end 143.9 88.5) (width 0.25) (locked yes) (layer "F.Cu") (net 6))
 (via (at 65.675 91.6) (size 0.6) (drill 0.3) (layers "F.Cu" "B.Cu") (locked yes) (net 6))
 (via (at 116.5 91.6) (size 0.6) (drill 0.3) (layers "F.Cu" "B.Cu") (locked yes) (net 6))
 (via (at 108.89 91.6) (size 0.6) (drill 0.3) (layers "F.Cu" "B.Cu") (locked yes) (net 6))
 (via (at 134.325 91.6) (size 0.6) (drill 0.3) (layers "F.Cu" "B.Cu") (locked yes) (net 6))
 (segment (start 65.675 91.6) (end 134.325 91.6) (width 0.25) (locked yes) (layer "B.Cu") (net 6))
 (segment (start 107.62 89.3) (end 113.775 89.3) (width 0.25) (locked yes) (layer "F.Cu") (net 15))
 (segment (start 107.62 94.3) (end 107.62 89.3) (width 0.25) (locked yes) (layer "F.Cu") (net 15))
 (via (at 107.62 94.3) (size 0.6) (drill 0.3) (layers "F.Cu" "B.Cu") (locked yes) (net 15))
 (segment (start 101.27 98.4) (end 112.9 98.4) (width 0.25) (locked yes) (layer "F.Cu") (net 11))
 (segment (start 112.9 98.4) (end 112.9 94.3) (width 0.25) (locked yes) (layer "F.Cu") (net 11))
 (segment (start 101.27 95.4) (end 101.27 98.4) (width 0.25) (locked yes) (layer "F.Cu") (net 11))
 (segment (start 112.9 98.4) (end 114.6 98.4) (width 0.25) (locked yes) (layer "F.Cu") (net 11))
 (via (at 112.9 94.3) (size 0.6) (drill 0.3) (layers "F.Cu" "B.Cu") (locked yes) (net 11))
 (segment (start 84.6 89.625) (end 84.6 88.65) (width 0.4) (locked yes) (layer "F.Cu") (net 4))
 (segment (start 79.6 90.45) (end 79.6 89) (width 0.5) (locked yes) (layer "F.Cu") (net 4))
 (segment (start 77.5 94.3) (end 77.5 89.4) (width 1.4) (locked yes) (layer "F.Cu") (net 4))
 (segment (start 86.775 97.95) (end 86.775 94.3) (width 0.3) (locked yes) (layer "F.Cu") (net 4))
 (segment (start 127.35 88.6) (end 129.1 88.6) (width 0.4) (locked yes) (layer "F.Cu") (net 4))
 (segment (start 122.1 94.3) (end 122.1 89.4) (width 1) (locked yes) (layer "F.Cu") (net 4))
 (segment (start 91.11 97.95) (end 86.775 97.95) (width 0.3) (locked yes) (layer "F.Cu") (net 4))
 (segment (start 91.11 95.4) (end 91.11 89) (width 0.5) (locked yes) (layer "F.Cu") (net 4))
 (segment (start 67.55 88.6) (end 69.3 88.6) (width 0.4) (locked yes) (layer "F.Cu") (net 4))
 (segment (start 91.11 95.4) (end 91.11 97.95) (width 0.3) (locked yes) (layer "F.Cu") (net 4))
 (segment (start 105.4 89.625) (end 105.4 88.65) (width 0.4) (locked yes) (layer "F.Cu") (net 4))
 (segment (start 86.775 94.3) (end 86.775 89.4) (width 1) (locked yes) (layer "F.Cu") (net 4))
 (segment (start 97.45 88.6) (end 99.2 88.6) (width 0.4) (locked yes) (layer "F.Cu") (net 4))
 (segment (start 119.8 89.625) (end 119.8 88.65) (width 0.4) (locked yes) (layer "F.Cu") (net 4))
 (via (at 122.5 89) (size 0.6) (drill 0.3) (layers "F.Cu" "B.Cu") (locked yes) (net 4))
 (via (at 86.4 94.3) (size 0.6) (drill 0.3) (layers "F.Cu" "B.Cu") (locked yes) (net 4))
 (via (at 105.4 88.65) (size 0.6) (drill 0.3) (layers "F.Cu" "B.Cu") (locked yes) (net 4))
 (via (at 121.7 89) (size 0.6) (drill 0.3) (layers "F.Cu" "B.Cu") (locked yes) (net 4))
 (via (at 79.6 89) (size 0.6) (drill 0.3) (layers "F.Cu" "B.Cu") (locked yes) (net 4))
 (via (at 119.8 88.65) (size 0.6) (drill 0.3) (layers "F.Cu" "B.Cu") (locked yes) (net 4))
 (via (at 84.6 88.65) (size 0.6) (drill 0.3) (layers "F.Cu" "B.Cu") (locked yes) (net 4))
 (via (at 78.3 89) (size 0.6) (drill 0.3) (layers "F.Cu" "B.Cu") (locked yes) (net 4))
 (via (at 77.5 89) (size 0.6) (drill 0.3) (layers "F.Cu" "B.Cu") (locked yes) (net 4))
 (via (at 87.15 94.3) (size 0.6) (drill 0.3) (layers "F.Cu" "B.Cu") (locked yes) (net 4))
 (via (at 76.7 89) (size 0.6) (drill 0.3) (layers "F.Cu" "B.Cu") (locked yes) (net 4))
 (via (at 91.11 89) (size 0.6) (drill 0.3) (layers "F.Cu" "B.Cu") (locked yes) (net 4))
 (via (at 78.3 94.3) (size 0.6) (drill 0.3) (layers "F.Cu" "B.Cu") (locked yes) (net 4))
 (via (at 77.5 94.3) (size 0.6) (drill 0.3) (layers "F.Cu" "B.Cu") (locked yes) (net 4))
 (via (at 87.15 89) (size 0.6) (drill 0.3) (layers "F.Cu" "B.Cu") (locked yes) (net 4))
 (via (at 121.7 94.3) (size 0.6) (drill 0.3) (layers "F.Cu" "B.Cu") (locked yes) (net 4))
 (via (at 76.7 94.3) (size 0.6) (drill 0.3) (layers "F.Cu" "B.Cu") (locked yes) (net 4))
 (via (at 69.3 88.6) (size 0.6) (drill 0.3) (layers "F.Cu" "B.Cu") (locked yes) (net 4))
 (via (at 99.2 88.6) (size 0.6) (drill 0.3) (layers "F.Cu" "B.Cu") (locked yes) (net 4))
 (via (at 129.1 88.6) (size 0.6) (drill 0.3) (layers "F.Cu" "B.Cu") (locked yes) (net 4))
 (via (at 122.5 94.3) (size 0.6) (drill 0.3) (layers "F.Cu" "B.Cu") (locked yes) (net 4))
 (via (at 86.4 89) (size 0.6) (drill 0.3) (layers "F.Cu" "B.Cu") (locked yes) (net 4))
 (segment (start 60.675 88.6) (end 139.325 88.6) (width 1.4) (locked yes) (layer "B.Cu") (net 4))
 (segment (start 60.675 92.75) (end 56.6 92.75) (width 1.2) (locked yes) (layer "B.Cu") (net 4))
 (segment (start 139.325 92.75) (end 143.4 92.75) (width 1.2) (locked yes) (layer "B.Cu") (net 4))
 (segment (start 60.675 88.6) (end 60.675 92.75) (width 1.2) (locked yes) (layer "B.Cu") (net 4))
 (segment (start 139.325 88.6) (end 139.325 92.75) (width 1.2) (locked yes) (layer "B.Cu") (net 4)))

